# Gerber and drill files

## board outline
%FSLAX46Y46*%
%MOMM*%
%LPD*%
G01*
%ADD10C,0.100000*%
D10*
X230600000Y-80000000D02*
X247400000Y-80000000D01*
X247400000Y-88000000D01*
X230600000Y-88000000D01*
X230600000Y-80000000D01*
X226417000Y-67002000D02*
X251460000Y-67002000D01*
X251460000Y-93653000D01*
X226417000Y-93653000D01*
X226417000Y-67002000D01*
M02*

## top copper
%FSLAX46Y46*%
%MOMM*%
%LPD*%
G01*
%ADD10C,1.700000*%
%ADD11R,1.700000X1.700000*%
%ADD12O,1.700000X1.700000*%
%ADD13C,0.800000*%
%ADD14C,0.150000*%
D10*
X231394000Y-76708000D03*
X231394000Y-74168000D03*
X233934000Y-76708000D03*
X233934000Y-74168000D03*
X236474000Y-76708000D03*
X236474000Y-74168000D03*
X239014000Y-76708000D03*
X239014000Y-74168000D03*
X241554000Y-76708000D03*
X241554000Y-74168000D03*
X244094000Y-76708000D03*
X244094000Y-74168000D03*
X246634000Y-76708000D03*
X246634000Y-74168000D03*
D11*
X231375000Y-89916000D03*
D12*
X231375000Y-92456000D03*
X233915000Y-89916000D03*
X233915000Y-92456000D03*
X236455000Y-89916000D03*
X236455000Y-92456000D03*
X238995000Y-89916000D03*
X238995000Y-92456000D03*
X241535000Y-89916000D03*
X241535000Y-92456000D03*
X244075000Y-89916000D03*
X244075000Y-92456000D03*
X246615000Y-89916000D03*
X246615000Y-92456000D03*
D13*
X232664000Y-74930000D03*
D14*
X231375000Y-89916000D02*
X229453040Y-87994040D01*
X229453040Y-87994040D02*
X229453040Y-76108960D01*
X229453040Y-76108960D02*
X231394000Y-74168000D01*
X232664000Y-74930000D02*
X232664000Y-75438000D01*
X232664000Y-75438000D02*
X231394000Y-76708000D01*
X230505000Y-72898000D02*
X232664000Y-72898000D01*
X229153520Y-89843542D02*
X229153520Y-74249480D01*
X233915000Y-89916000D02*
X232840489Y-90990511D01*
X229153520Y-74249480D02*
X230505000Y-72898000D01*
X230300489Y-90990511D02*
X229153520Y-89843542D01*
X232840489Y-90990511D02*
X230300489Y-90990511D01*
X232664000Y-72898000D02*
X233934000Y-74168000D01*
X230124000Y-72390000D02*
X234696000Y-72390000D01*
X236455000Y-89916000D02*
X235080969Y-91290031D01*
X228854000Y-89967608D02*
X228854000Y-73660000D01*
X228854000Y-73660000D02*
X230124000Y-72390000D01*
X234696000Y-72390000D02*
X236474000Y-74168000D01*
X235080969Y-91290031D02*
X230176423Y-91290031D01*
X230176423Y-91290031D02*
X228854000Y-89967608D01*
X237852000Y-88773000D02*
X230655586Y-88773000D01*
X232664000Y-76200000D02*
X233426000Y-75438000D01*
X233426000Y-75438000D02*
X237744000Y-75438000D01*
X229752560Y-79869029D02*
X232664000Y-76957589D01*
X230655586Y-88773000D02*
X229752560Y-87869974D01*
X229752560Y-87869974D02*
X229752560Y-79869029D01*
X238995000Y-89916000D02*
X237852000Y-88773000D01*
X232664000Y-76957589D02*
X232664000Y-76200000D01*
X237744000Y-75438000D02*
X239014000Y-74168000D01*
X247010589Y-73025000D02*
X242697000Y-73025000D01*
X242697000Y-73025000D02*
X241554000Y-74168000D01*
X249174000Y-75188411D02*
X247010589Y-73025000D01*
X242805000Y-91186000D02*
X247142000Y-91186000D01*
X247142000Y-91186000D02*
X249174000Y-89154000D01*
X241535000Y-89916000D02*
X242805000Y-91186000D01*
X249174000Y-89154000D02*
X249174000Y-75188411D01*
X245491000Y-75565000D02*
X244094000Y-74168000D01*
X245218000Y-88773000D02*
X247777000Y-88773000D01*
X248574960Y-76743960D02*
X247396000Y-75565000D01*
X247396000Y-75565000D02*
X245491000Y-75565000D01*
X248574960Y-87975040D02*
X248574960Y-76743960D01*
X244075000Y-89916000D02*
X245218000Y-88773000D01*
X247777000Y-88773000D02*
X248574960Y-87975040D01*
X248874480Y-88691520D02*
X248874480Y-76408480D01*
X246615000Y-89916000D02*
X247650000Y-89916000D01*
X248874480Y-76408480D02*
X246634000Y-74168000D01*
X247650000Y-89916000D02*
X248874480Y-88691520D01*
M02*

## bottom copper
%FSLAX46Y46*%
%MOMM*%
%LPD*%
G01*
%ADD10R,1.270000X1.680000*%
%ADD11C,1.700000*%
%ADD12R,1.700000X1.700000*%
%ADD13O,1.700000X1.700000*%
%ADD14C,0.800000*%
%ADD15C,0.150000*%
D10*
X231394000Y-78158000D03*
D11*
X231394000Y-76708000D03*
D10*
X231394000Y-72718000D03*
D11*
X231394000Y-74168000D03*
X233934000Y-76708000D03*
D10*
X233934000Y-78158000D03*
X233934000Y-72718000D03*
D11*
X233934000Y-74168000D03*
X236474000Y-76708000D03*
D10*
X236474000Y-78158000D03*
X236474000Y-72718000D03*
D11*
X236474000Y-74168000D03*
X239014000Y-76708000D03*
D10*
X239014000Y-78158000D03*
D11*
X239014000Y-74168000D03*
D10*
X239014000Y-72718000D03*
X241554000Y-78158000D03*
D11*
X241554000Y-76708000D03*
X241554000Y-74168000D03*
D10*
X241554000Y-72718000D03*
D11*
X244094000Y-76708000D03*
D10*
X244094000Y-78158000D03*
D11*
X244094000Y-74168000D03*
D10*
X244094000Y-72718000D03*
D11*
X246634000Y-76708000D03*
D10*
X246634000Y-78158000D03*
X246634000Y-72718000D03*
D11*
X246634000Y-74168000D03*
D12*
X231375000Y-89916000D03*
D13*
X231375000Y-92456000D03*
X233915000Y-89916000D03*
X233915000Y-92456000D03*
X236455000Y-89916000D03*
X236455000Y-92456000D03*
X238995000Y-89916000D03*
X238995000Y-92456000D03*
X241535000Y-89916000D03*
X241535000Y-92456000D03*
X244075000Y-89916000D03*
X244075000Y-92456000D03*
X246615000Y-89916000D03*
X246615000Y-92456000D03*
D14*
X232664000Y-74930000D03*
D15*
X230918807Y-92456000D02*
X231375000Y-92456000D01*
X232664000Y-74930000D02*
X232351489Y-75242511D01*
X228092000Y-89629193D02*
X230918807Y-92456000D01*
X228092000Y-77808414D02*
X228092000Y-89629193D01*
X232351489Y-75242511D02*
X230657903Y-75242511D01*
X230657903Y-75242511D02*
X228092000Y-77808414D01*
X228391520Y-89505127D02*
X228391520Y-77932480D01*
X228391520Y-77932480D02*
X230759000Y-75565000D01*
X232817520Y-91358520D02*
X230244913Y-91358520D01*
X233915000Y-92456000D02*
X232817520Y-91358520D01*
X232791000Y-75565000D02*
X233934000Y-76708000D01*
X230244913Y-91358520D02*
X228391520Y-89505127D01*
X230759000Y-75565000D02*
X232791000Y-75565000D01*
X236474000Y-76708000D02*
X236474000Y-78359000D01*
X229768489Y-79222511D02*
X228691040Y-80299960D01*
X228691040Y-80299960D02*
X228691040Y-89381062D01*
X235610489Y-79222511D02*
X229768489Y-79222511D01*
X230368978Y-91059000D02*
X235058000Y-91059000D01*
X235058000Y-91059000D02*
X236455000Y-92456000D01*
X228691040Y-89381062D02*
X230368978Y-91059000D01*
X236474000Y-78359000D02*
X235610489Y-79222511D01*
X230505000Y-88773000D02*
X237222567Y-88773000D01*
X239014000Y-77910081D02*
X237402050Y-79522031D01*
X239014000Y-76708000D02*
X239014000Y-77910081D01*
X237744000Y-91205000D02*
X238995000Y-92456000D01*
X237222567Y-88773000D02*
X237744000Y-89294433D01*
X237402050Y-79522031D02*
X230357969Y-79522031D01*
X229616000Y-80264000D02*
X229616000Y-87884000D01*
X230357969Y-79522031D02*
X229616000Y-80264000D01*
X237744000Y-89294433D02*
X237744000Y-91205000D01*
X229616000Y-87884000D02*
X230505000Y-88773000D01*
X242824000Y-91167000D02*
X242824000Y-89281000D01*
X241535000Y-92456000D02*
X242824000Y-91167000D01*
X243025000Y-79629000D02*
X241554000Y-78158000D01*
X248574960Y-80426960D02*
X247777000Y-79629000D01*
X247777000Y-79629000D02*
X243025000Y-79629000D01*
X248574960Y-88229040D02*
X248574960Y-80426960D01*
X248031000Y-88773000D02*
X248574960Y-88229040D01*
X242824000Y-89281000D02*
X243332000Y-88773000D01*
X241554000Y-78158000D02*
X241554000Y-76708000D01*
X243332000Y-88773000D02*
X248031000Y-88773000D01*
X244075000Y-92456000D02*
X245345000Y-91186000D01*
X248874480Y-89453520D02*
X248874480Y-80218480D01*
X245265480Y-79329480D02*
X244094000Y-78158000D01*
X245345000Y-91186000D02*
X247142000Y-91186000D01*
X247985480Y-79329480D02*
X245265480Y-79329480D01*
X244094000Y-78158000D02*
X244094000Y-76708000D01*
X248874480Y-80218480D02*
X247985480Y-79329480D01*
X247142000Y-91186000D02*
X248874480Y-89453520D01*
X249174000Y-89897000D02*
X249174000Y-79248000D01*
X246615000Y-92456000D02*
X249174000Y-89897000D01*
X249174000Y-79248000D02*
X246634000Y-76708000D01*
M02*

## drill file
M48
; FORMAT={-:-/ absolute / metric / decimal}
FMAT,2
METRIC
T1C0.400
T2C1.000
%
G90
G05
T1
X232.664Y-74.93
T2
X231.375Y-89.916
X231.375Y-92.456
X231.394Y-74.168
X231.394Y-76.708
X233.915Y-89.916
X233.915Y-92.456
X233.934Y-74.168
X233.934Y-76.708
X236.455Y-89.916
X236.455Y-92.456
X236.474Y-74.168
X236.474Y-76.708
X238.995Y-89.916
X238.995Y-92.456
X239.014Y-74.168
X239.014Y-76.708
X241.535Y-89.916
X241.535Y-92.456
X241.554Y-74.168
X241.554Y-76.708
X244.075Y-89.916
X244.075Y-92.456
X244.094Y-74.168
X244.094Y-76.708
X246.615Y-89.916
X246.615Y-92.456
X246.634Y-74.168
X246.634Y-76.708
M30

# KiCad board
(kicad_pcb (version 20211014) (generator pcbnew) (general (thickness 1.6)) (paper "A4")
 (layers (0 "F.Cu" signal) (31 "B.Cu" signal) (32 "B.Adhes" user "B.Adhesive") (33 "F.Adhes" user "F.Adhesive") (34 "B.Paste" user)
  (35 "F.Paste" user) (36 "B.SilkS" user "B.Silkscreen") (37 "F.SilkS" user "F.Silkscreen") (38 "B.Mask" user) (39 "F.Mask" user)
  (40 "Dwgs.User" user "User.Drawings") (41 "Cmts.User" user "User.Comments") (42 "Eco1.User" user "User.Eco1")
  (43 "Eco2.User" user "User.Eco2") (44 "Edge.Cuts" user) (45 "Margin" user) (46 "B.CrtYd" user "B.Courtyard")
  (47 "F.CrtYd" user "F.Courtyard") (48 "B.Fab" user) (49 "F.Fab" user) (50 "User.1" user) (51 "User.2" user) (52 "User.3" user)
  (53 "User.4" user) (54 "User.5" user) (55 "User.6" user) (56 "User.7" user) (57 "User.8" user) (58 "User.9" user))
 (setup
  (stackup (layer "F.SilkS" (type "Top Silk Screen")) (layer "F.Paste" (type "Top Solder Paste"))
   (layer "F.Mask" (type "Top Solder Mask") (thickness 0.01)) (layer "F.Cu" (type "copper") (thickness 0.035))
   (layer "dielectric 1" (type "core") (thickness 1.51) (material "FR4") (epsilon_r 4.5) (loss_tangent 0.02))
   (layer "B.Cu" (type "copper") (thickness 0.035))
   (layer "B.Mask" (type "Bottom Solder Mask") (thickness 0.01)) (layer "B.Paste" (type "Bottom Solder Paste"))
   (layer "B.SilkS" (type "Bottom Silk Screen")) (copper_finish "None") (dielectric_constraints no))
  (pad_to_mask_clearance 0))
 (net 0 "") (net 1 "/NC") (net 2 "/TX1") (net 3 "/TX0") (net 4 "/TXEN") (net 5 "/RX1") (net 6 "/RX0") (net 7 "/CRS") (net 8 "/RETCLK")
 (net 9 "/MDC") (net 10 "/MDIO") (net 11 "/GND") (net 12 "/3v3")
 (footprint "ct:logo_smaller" (layer "F.Cu") (at 245.872 70.485)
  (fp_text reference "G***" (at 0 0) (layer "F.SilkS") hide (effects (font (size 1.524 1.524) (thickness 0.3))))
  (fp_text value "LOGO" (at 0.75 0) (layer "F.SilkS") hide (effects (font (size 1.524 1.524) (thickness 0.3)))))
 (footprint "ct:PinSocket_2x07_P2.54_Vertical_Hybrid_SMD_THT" (layer "B.Cu") (at 239.014 71.378)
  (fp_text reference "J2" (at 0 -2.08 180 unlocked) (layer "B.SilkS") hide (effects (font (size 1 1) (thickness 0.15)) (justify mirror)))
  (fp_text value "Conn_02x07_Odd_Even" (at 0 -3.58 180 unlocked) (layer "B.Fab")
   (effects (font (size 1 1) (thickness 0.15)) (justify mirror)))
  (pad "1" smd rect (at -7.62 6.78) (size 1.27 1.68) (layers "B.Cu" "B.Paste" "B.Mask") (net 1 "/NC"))
  (pad "1" thru_hole circle (at -7.62 5.33) (size 1.7 1.7) (drill 1) (layers *.Cu *.Mask) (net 1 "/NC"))
  (pad "2" smd rect (at -7.62 1.34) (size 1.27 1.68) (layers "B.Cu" "B.Paste" "B.Mask") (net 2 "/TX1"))
  (pad "2" thru_hole circle (at -7.62 2.79) (size 1.7 1.7) (drill 1) (layers *.Cu *.Mask) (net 2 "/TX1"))
  (pad "3" thru_hole circle (at -5.08 5.33) (size 1.7 1.7) (drill 1) (layers *.Cu *.Mask) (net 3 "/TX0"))
  (pad "3" smd rect (at -5.08 6.78) (size 1.27 1.68) (layers "B.Cu" "B.Paste" "B.Mask") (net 3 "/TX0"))
  (pad "4" smd rect (at -5.08 1.34) (size 1.27 1.68) (layers "B.Cu" "B.Paste" "B.Mask") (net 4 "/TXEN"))
  (pad "4" thru_hole circle (at -5.08 2.79) (size 1.7 1.7) (drill 1) (layers *.Cu *.Mask) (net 4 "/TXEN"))
  (pad "5" thru_hole circle (at -2.54 5.33) (size 1.7 1.7) (drill 1) (layers *.Cu *.Mask) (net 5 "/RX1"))
  (pad "5" smd rect (at -2.54 6.78) (size 1.27 1.68) (layers "B.Cu" "B.Paste" "B.Mask") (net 5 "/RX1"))
  (pad "6" smd rect (at -2.54 1.34) (size 1.27 1.68) (layers "B.Cu" "B.Paste" "B.Mask") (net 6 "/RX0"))
  (pad "6" thru_hole circle (at -2.54 2.79) (size 1.7 1.7) (drill 1) (layers *.Cu *.Mask) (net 6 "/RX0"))
  (pad "7" thru_hole circle (at 0 5.33) (size 1.7 1.7) (drill 1) (layers *.Cu *.Mask) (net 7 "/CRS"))
  (pad "7" smd rect (at 0 6.78) (size 1.27 1.68) (layers "B.Cu" "B.Paste" "B.Mask") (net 7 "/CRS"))
  (pad "8" thru_hole circle (at 0 2.79) (size 1.7 1.7) (drill 1) (layers *.Cu *.Mask) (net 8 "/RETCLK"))
  (pad "8" smd rect (at 0 1.34) (size 1.27 1.68) (layers "B.Cu" "B.Paste" "B.Mask") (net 8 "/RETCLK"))
  (pad "9" smd rect (at 2.54 6.78) (size 1.27 1.68) (layers "B.Cu" "B.Paste" "B.Mask") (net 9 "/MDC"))
  (pad "9" thru_hole circle (at 2.54 5.33) (size 1.7 1.7) (drill 1) (layers *.Cu *.Mask) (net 9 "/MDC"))
  (pad "10" thru_hole circle (at 2.54 2.79) (size 1.7 1.7) (drill 1) (layers *.Cu *.Mask) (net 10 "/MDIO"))
  (pad "10" smd rect (at 2.54 1.34) (size 1.27 1.68) (layers "B.Cu" "B.Paste" "B.Mask") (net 10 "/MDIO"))
  (pad "11" thru_hole circle (at 5.08 5.33) (size 1.7 1.7) (drill 1) (layers *.Cu *.Mask) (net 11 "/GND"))
  (pad "11" smd rect (at 5.08 6.78) (size 1.27 1.68) (layers "B.Cu" "B.Paste" "B.Mask") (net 11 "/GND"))
  (pad "12" thru_hole circle (at 5.08 2.79) (size 1.7 1.7) (drill 1) (layers *.Cu *.Mask) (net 11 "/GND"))
  (pad "12" smd rect (at 5.08 1.34) (size 1.27 1.68) (layers "B.Cu" "B.Paste" "B.Mask") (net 11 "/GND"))
  (pad "13" thru_hole circle (at 7.62 5.33) (size 1.7 1.7) (drill 1) (layers *.Cu *.Mask) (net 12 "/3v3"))
  (pad "13" smd rect (at 7.62 6.78) (size 1.27 1.68) (layers "B.Cu" "B.Paste" "B.Mask") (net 12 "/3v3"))
  (pad "14" smd rect (at 7.62 1.34) (size 1.27 1.68) (layers "B.Cu" "B.Paste" "B.Mask") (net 12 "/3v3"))
  (pad "14" thru_hole circle (at 7.62 2.79) (size 1.7 1.7) (drill 1) (layers *.Cu *.Mask) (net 12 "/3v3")))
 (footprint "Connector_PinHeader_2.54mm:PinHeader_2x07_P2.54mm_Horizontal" (layer "B.Cu") (at 231.375 89.916 -90) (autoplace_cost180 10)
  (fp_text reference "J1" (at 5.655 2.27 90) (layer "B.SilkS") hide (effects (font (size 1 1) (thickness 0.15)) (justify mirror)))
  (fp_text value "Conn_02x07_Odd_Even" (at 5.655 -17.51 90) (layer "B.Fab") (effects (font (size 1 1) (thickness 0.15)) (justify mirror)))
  (pad "1" thru_hole rect (at 0 0 270) (size 1.7 1.7) (drill 1) (layers *.Cu *.Mask) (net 2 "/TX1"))
  (pad "2" thru_hole oval (at 2.54 0 270) (size 1.7 1.7) (drill 1) (layers *.Cu *.Mask) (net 1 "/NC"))
  (pad "3" thru_hole oval (at 0 -2.54 270) (size 1.7 1.7) (drill 1) (layers *.Cu *.Mask) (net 4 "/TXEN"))
  (pad "4" thru_hole oval (at 2.54 -2.54 270) (size 1.7 1.7) (drill 1) (layers *.Cu *.Mask) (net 3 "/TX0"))
  (pad "5" thru_hole oval (at 0 -5.08 270) (size 1.7 1.7) (drill 1) (layers *.Cu *.Mask) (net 6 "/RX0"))
  (pad "6" thru_hole oval (at 2.54 -5.08 270) (size 1.7 1.7) (drill 1) (layers *.Cu *.Mask) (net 5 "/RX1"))
  (pad "7" thru_hole oval (at 0 -7.62 270) (size 1.7 1.7) (drill 1) (layers *.Cu *.Mask) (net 8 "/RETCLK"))
  (pad "8" thru_hole oval (at 2.54 -7.62 270) (size 1.7 1.7) (drill 1) (layers *.Cu *.Mask) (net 7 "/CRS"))
  (pad "9" thru_hole oval (at 0 -10.16 270) (size 1.7 1.7) (drill 1) (layers *.Cu *.Mask) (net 10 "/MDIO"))
  (pad "10" thru_hole oval (at 2.54 -10.16 270) (size 1.7 1.7) (drill 1) (layers *.Cu *.Mask) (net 9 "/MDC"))
  (pad "11" thru_hole oval (at 0 -12.7 270) (size 1.7 1.7) (drill 1) (layers *.Cu *.Mask) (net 11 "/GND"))
  (pad "12" thru_hole oval (at 2.54 -12.7 270) (size 1.7 1.7) (drill 1) (layers *.Cu *.Mask) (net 11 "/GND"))
  (pad "13" thru_hole oval (at 0 -15.24 270) (size 1.7 1.7) (drill 1) (layers *.Cu *.Mask) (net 12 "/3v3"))
  (pad "14" thru_hole oval (at 2.54 -15.24 270) (size 1.7 1.7) (drill 1) (layers *.Cu *.Mask) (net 12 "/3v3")))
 (gr_rect (start 230.6 80) (end 247.4 88) (layer "Edge.Cuts") (width 0.1) (fill none))
 (gr_rect (start 226.417 67.002) (end 251.46 93.653) (layer "Edge.Cuts") (width 0.1) (fill none))
 (segment (start 231.375 89.916) (end 229.45304 87.99404) (width 0.15) (layer "F.Cu") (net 2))
 (segment (start 229.45304 87.99404) (end 229.45304 76.10896) (width 0.15) (layer "F.Cu") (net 2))
 (segment (start 229.45304 76.10896) (end 231.394 74.168) (width 0.15) (layer "F.Cu") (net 2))
 (segment (start 232.664 74.93) (end 232.664 75.438) (width 0.15) (layer "F.Cu") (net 1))
 (segment (start 232.664 75.438) (end 231.394 76.708) (width 0.15) (layer "F.Cu") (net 1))
 (via (at 232.664 74.93) (size 0.8) (drill 0.4) (layers "F.Cu" "B.Cu") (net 1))
 (segment (start 230.918807 92.456) (end 231.375 92.456) (width 0.15) (layer "B.Cu") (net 1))
 (segment (start 232.664 74.93) (end 232.351489 75.242511) (width 0.15) (layer "B.Cu") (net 1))
 (segment (start 228.092 89.629193) (end 230.918807 92.456) (width 0.15) (layer "B.Cu") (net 1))
 (segment (start 228.092 77.808414) (end 228.092 89.629193) (width 0.15) (layer "B.Cu") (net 1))
 (segment (start 232.351489 75.242511) (end 230.657903 75.242511) (width 0.15) (layer "B.Cu") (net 1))
 (segment (start 230.657903 75.242511) (end 228.092 77.808414) (width 0.15) (layer "B.Cu") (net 1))
 (segment (start 230.505 72.898) (end 232.664 72.898) (width 0.15) (layer "F.Cu") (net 4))
 (segment (start 229.15352 89.843542) (end 229.15352 74.24948) (width 0.15) (layer "F.Cu") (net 4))
 (segment (start 233.915 89.916) (end 232.840489 90.990511) (width 0.15) (layer "F.Cu") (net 4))
 (segment (start 229.15352 74.24948) (end 230.505 72.898) (width 0.15) (layer "F.Cu") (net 4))
 (segment (start 230.300489 90.990511) (end 229.15352 89.843542) (width 0.15) (layer "F.Cu") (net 4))
 (segment (start 232.840489 90.990511) (end 230.300489 90.990511) (width 0.15) (layer "F.Cu") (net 4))
 (segment (start 232.664 72.898) (end 233.934 74.168) (width 0.15) (layer "F.Cu") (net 4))
 (segment (start 228.39152 89.505127) (end 228.39152 77.93248) (width 0.15) (layer "B.Cu") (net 3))
 (segment (start 228.39152 77.93248) (end 230.759 75.565) (width 0.15) (layer "B.Cu") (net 3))
 (segment (start 232.81752 91.35852) (end 230.244913 91.35852) (width 0.15) (layer "B.Cu") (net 3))
 (segment (start 233.915 92.456) (end 232.81752 91.35852) (width 0.15) (layer "B.Cu") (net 3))
 (segment (start 232.791 75.565) (end 233.934 76.708) (width 0.15) (layer "B.Cu") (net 3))
 (segment (start 230.244913 91.35852) (end 228.39152 89.505127) (width 0.15) (layer "B.Cu") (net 3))
 (segment (start 230.759 75.565) (end 232.791 75.565) (width 0.15) (layer "B.Cu") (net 3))
 (segment (start 230.124 72.39) (end 234.696 72.39) (width 0.15) (layer "F.Cu") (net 6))
 (segment (start 236.455 89.916) (end 235.080969 91.290031) (width 0.15) (layer "F.Cu") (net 6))
 (segment (start 228.854 89.967608) (end 228.854 73.66) (width 0.15) (layer "F.Cu") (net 6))
 (segment (start 228.854 73.66) (end 230.124 72.39) (width 0.15) (layer "F.Cu") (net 6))
 (segment (start 234.696 72.39) (end 236.474 74.168) (width 0.15) (layer "F.Cu") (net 6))
 (segment (start 235.080969 91.290031) (end 230.176423 91.290031) (width 0.15) (layer "F.Cu") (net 6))
 (segment (start 230.176423 91.290031) (end 228.854 89.967608) (width 0.15) (layer "F.Cu") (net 6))
 (segment (start 236.474 76.708) (end 236.474 78.359) (width 0.15) (layer "B.Cu") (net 5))
 (segment (start 229.768489 79.222511) (end 228.69104 80.29996) (width 0.15) (layer "B.Cu") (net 5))
 (segment (start 228.69104 80.29996) (end 228.69104 89.381062) (width 0.15) (layer "B.Cu") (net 5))
 (segment (start 235.610489 79.222511) (end 229.768489 79.222511) (width 0.15) (layer "B.Cu") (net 5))
 (segment (start 230.368978 91.059) (end 235.058 91.059) (width 0.15) (layer "B.Cu") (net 5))
 (segment (start 235.058 91.059) (end 236.455 92.456) (width 0.15) (layer "B.Cu") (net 5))
 (segment (start 228.69104 89.381062) (end 230.368978 91.059) (width 0.15) (layer "B.Cu") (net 5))
 (segment (start 236.474 78.359) (end 235.610489 79.222511) (width 0.15) (layer "B.Cu") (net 5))
 (segment (start 237.852 88.773) (end 230.655586 88.773) (width 0.15) (layer "F.Cu") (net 8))
 (segment (start 232.664 76.2) (end 233.426 75.438) (width 0.15) (layer "F.Cu") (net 8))
 (segment (start 233.426 75.438) (end 237.744 75.438) (width 0.15) (layer "F.Cu") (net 8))
 (segment (start 229.75256 79.869029) (end 232.664 76.957589) (width 0.15) (layer "F.Cu") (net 8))
 (segment (start 230.655586 88.773) (end 229.75256 87.869974) (width 0.15) (layer "F.Cu") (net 8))
 (segment (start 229.75256 87.869974) (end 229.75256 79.869029) (width 0.15) (layer "F.Cu") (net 8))
 (segment (start 238.995 89.916) (end 237.852 88.773) (width 0.15) (layer "F.Cu") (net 8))
 (segment (start 232.664 76.957589) (end 232.664 76.2) (width 0.15) (layer "F.Cu") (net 8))
 (segment (start 237.744 75.438) (end 239.014 74.168) (width 0.15) (layer "F.Cu") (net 8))
 (segment (start 230.505 88.773) (end 237.222567 88.773) (width 0.15) (layer "B.Cu") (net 7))
 (segment (start 239.014 77.910081) (end 237.40205 79.522031) (width 0.15) (layer "B.Cu") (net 7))
 (segment (start 239.014 76.708) (end 239.014 77.910081) (width 0.15) (layer "B.Cu") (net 7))
 (segment (start 237.744 91.205) (end 238.995 92.456) (width 0.15) (layer "B.Cu") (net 7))
 (segment (start 237.222567 88.773) (end 237.744 89.294433) (width 0.15) (layer "B.Cu") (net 7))
 (segment (start 237.40205 79.522031) (end 230.357969 79.522031) (width 0.15) (layer "B.Cu") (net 7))
 (segment (start 229.616 80.264) (end 229.616 87.884) (width 0.15) (layer "B.Cu") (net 7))
 (segment (start 230.357969 79.522031) (end 229.616 80.264) (width 0.15) (layer "B.Cu") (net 7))
 (segment (start 237.744 89.294433) (end 237.744 91.205) (width 0.15) (layer "B.Cu") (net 7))
 (segment (start 229.616 87.884) (end 230.505 88.773) (width 0.15) (layer "B.Cu") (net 7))
 (segment (start 247.010589 73.025) (end 242.697 73.025) (width 0.15) (layer "F.Cu") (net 10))
 (segment (start 242.697 73.025) (end 241.554 74.168) (width 0.15) (layer "F.Cu") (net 10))
 (segment (start 249.174 75.188411) (end 247.010589 73.025) (width 0.15) (layer "F.Cu") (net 10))
 (segment (start 242.805 91.186) (end 247.142 91.186) (width 0.15) (layer "F.Cu") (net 10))
 (segment (start 247.142 91.186) (end 249.174 89.154) (width 0.15) (layer "F.Cu") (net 10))
 (segment (start 241.535 89.916) (end 242.805 91.186) (width 0.15) (layer "F.Cu") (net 10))
 (segment (start 249.174 89.154) (end 249.174 75.188411) (width 0.15) (layer "F.Cu") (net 10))
 (segment (start 242.824 91.167) (end 242.824 89.281) (width 0.15) (layer "B.Cu") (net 9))
 (segment (start 241.535 92.456) (end 242.824 91.167) (width 0.15) (layer "B.Cu") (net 9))
 (segment (start 243.025 79.629) (end 241.554 78.158) (width 0.15) (layer "B.Cu") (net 9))
 (segment (start 248.57496 80.42696) (end 247.777 79.629) (width 0.15) (layer "B.Cu") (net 9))
 (segment (start 247.777 79.629) (end 243.025 79.629) (width 0.15) (layer "B.Cu") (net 9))
 (segment (start 248.57496 88.22904) (end 248.57496 80.42696) (width 0.15) (layer "B.Cu") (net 9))
 (segment (start 248.031 88.773) (end 248.57496 88.22904) (width 0.15) (layer "B.Cu") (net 9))
 (segment (start 242.824 89.281) (end 243.332 88.773) (width 0.15) (layer "B.Cu") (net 9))
 (segment (start 241.554 78.158) (end 241.554 76.708) (width 0.15) (layer "B.Cu") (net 9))
 (segment (start 243.332 88.773) (end 248.031 88.773) (width 0.15) (layer "B.Cu") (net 9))
 (segment (start 245.491 75.565) (end 244.094 74.168) (width 0.15) (layer "F.Cu") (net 11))
 (segment (start 245.218 88.773) (end 247.777 88.773) (width 0.15) (layer "F.Cu") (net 11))
 (segment (start 248.57496 76.74396) (end 247.396 75.565) (width 0.15) (layer "F.Cu") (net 11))
 (segment (start 247.396 75.565) (end 245.491 75.565) (width 0.15) (layer "F.Cu") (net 11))
 (segment (start 248.57496 87.97504) (end 248.57496 76.74396) (width 0.15) (layer "F.Cu") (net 11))
 (segment (start 244.075 89.916) (end 245.218 88.773) (width 0.15) (layer "F.Cu") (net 11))
 (segment (start 247.777 88.773) (end 248.57496 87.97504) (width 0.15) (layer "F.Cu") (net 11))
 (segment (start 244.075 92.456) (end 245.345 91.186) (width 0.15) (layer "B.Cu") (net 11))
 (segment (start 248.87448 89.45352) (end 248.87448 80.21848) (width 0.15) (layer "B.Cu") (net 11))
 (segment (start 245.26548 79.32948) (end 244.094 78.158) (width 0.15) (layer "B.Cu") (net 11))
 (segment (start 245.345 91.186) (end 247.142 91.186) (width 0.15) (layer "B.Cu") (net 11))
 (segment (start 247.98548 79.32948) (end 245.26548 79.32948) (width 0.15) (layer "B.Cu") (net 11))
 (segment (start 244.094 78.158) (end 244.094 76.708) (width 0.15) (layer "B.Cu") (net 11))
 (segment (start 248.87448 80.21848) (end 247.98548 79.32948) (width 0.15) (layer "B.Cu") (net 11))
 (segment (start 247.142 91.186) (end 248.87448 89.45352) (width 0.15) (layer "B.Cu") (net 11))
 (segment (start 248.87448 88.69152) (end 248.87448 76.40848) (width 0.15) (layer "F.Cu") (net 12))
 (segment (start 246.615 89.916) (end 247.65 89.916) (width 0.15) (layer "F.Cu") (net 12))
 (segment (start 248.87448 76.40848) (end 246.634 74.168) (width 0.15) (layer "F.Cu") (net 12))
 (segment (start 247.65 89.916) (end 248.87448 88.69152) (width 0.15) (layer "F.Cu") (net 12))
 (segment (start 249.174 89.897) (end 249.174 79.248) (width 0.15) (layer "B.Cu") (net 12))
 (segment (start 246.615 92.456) (end 249.174 89.897) (width 0.15) (layer "B.Cu") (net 12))
 (segment (start 249.174 79.248) (end 246.634 76.708) (width 0.15) (layer "B.Cu") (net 12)))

